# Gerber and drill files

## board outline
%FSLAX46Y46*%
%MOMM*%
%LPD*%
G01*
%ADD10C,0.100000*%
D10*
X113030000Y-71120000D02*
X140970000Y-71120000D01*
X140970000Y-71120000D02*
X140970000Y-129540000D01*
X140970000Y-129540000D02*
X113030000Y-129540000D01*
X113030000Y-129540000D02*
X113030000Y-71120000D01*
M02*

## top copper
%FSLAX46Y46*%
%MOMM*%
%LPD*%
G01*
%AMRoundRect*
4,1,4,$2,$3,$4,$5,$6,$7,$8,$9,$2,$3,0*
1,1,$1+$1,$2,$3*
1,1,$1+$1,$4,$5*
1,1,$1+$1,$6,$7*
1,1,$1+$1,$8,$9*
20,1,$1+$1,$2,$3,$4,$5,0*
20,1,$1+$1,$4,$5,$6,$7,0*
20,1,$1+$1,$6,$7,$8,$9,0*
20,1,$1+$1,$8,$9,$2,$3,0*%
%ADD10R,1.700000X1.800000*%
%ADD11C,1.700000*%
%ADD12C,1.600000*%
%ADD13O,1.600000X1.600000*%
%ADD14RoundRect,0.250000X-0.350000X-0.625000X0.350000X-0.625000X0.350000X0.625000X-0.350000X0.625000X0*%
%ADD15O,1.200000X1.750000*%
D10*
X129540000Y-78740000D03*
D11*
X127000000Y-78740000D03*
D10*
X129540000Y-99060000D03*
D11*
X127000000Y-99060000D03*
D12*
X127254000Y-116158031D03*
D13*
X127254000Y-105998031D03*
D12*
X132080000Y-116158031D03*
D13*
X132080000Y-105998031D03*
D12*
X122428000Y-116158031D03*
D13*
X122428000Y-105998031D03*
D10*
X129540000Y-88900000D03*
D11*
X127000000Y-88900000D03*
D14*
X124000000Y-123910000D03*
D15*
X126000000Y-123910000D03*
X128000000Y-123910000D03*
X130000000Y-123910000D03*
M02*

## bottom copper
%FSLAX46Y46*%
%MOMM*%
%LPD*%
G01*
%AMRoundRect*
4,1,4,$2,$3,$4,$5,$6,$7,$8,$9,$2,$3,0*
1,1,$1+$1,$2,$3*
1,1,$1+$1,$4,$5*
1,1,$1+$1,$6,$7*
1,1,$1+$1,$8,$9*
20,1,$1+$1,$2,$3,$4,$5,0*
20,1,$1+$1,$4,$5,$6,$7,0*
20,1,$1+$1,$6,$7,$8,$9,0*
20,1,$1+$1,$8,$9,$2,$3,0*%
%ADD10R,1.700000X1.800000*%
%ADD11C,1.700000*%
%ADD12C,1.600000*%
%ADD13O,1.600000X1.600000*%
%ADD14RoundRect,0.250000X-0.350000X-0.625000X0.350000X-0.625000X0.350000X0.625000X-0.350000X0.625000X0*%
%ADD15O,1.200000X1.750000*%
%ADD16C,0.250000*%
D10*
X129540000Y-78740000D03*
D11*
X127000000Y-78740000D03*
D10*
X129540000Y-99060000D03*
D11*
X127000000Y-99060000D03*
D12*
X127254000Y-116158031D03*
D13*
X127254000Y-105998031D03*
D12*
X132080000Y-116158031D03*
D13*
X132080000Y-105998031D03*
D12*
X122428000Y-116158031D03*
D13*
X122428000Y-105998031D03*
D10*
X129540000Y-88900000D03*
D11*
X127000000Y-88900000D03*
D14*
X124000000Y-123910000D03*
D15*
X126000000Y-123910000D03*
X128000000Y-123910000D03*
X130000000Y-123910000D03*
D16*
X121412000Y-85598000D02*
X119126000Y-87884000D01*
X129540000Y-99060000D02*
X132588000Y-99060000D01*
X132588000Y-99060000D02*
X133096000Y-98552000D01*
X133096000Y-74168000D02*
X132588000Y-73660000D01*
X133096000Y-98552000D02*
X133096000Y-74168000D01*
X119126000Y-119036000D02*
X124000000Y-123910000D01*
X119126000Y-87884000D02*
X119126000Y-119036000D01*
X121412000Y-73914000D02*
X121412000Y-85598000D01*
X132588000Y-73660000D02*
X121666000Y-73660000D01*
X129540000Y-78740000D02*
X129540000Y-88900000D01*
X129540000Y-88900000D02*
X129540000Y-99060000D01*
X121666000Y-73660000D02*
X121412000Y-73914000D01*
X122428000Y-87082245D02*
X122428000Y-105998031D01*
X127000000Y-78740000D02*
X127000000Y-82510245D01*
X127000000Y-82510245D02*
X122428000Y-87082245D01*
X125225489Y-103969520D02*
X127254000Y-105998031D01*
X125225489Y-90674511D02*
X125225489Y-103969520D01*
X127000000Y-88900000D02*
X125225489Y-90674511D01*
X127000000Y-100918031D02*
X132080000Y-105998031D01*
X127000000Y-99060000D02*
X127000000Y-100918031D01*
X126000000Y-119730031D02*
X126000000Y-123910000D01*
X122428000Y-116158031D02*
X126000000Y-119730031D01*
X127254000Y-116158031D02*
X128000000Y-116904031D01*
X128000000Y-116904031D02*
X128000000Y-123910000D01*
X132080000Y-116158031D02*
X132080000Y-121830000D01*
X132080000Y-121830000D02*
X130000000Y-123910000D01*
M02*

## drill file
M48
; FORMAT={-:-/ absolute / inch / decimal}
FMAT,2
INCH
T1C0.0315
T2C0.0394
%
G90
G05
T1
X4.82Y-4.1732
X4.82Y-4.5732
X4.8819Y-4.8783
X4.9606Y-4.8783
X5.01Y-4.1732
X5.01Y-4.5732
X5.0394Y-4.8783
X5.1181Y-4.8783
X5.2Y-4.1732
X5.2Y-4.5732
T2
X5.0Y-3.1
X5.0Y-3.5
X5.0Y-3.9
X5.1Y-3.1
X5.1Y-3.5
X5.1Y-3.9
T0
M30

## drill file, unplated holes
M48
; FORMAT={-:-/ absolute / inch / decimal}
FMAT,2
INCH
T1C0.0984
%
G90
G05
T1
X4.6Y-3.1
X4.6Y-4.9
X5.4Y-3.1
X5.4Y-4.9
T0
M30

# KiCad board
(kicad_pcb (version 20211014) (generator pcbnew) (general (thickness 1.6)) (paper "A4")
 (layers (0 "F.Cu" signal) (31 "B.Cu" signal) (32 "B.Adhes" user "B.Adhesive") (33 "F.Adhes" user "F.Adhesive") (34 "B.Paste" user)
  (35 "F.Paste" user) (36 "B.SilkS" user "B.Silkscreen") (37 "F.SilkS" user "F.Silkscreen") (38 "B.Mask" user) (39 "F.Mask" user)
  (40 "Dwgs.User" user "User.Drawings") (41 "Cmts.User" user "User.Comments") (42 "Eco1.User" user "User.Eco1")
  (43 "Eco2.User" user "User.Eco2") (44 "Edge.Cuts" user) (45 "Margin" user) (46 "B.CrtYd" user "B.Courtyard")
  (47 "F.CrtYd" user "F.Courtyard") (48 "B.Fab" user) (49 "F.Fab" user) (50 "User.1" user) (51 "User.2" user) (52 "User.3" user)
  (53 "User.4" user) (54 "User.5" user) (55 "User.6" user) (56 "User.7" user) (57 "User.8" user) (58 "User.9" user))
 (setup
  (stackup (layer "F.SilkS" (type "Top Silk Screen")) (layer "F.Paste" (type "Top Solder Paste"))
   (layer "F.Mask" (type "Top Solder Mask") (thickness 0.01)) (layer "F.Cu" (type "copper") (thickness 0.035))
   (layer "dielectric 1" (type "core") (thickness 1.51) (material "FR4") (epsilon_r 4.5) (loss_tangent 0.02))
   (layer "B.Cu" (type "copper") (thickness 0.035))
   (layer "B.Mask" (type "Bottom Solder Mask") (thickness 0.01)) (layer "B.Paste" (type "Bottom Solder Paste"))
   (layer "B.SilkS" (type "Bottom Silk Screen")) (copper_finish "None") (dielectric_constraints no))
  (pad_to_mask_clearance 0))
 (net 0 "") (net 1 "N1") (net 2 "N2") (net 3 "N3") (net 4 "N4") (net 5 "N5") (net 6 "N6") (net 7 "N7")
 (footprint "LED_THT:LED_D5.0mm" (layer "F.Cu") (at 129.54 78.74 180)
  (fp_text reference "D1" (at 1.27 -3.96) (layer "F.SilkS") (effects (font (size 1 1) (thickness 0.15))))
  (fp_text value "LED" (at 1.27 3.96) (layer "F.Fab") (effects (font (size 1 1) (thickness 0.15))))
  (pad "1" thru_hole rect (at 0 0 180) (size 1.7 1.8) (drill 1) (layers *.Cu *.Mask) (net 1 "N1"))
  (pad "2" thru_hole circle (at 2.54 0 180) (size 1.7 1.7) (drill 1) (layers *.Cu *.Mask) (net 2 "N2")))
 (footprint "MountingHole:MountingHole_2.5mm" (layer "F.Cu") (at 137.16 124.46)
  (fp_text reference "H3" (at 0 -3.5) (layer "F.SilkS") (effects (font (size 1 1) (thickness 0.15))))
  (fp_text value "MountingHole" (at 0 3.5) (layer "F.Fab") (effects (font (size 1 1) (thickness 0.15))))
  (pad "" np_thru_hole circle (at 0 0) (size 2.5 2.5) (drill 2.5) (layers *.Cu *.Mask)))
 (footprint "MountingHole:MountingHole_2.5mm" (layer "F.Cu") (at 137.16 78.74)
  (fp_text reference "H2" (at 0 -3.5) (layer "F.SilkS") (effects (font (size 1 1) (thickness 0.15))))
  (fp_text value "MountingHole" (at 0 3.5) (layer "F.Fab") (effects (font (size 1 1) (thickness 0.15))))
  (pad "" np_thru_hole circle (at 0 0) (size 2.5 2.5) (drill 2.5) (layers *.Cu *.Mask)))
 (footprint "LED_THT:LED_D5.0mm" (layer "F.Cu") (at 129.54 99.06 180)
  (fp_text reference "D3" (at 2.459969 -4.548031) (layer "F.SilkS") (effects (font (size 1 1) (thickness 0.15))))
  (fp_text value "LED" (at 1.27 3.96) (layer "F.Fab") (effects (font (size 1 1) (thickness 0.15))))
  (pad "1" thru_hole rect (at 0 0 180) (size 1.7 1.8) (drill 1) (layers *.Cu *.Mask) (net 1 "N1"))
  (pad "2" thru_hole circle (at 2.54 0 180) (size 1.7 1.7) (drill 1) (layers *.Cu *.Mask) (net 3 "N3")))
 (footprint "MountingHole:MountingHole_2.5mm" (layer "F.Cu") (at 116.84 124.46)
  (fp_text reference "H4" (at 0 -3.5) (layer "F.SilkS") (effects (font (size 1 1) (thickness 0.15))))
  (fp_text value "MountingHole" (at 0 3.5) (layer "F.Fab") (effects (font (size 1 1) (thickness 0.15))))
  (pad "" np_thru_hole circle (at 0 0) (size 2.5 2.5) (drill 2.5) (layers *.Cu *.Mask)))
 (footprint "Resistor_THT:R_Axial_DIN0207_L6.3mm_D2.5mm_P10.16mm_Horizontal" (layer "F.Cu") (at 127.254 116.158031 90)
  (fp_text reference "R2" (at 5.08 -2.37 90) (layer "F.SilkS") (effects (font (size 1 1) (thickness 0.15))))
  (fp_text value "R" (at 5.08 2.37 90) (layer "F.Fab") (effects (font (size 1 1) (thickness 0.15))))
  (pad "1" thru_hole circle (at 0 0 90) (size 1.6 1.6) (drill 0.8) (layers *.Cu *.Mask) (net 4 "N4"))
  (pad "2" thru_hole oval (at 10.16 0 90) (size 1.6 1.6) (drill 0.8) (layers *.Cu *.Mask) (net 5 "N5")))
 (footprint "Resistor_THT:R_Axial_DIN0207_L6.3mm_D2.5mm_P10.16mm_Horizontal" (layer "F.Cu") (at 132.08 116.158031 90)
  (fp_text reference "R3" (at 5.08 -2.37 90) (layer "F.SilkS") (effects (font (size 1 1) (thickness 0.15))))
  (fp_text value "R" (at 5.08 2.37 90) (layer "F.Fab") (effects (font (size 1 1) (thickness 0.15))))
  (pad "1" thru_hole circle (at 0 0 90) (size 1.6 1.6) (drill 0.8) (layers *.Cu *.Mask) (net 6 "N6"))
  (pad "2" thru_hole oval (at 10.16 0 90) (size 1.6 1.6) (drill 0.8) (layers *.Cu *.Mask) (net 3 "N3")))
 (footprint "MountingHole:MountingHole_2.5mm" (layer "F.Cu") (at 116.84 78.74)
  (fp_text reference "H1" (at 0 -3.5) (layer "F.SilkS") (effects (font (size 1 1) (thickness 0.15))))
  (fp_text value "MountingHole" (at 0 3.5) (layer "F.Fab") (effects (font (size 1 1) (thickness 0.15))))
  (pad "" np_thru_hole circle (at 0 0) (size 2.5 2.5) (drill 2.5) (layers *.Cu *.Mask)))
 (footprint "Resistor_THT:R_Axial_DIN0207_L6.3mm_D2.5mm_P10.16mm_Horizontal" (layer "F.Cu") (at 122.428 116.158031 90)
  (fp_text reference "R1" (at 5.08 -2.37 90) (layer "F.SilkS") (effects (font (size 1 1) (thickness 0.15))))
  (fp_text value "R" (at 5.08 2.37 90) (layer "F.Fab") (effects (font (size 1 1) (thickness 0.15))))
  (pad "1" thru_hole circle (at 0 0 90) (size 1.6 1.6) (drill 0.8) (layers *.Cu *.Mask) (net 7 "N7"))
  (pad "2" thru_hole oval (at 10.16 0 90) (size 1.6 1.6) (drill 0.8) (layers *.Cu *.Mask) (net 2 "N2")))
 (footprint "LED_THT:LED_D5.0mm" (layer "F.Cu") (at 129.54 88.9 180)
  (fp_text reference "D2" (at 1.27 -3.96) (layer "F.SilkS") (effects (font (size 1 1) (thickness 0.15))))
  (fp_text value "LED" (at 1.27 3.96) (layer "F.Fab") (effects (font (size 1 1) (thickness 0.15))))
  (pad "1" thru_hole rect (at 0 0 180) (size 1.7 1.8) (drill 1) (layers *.Cu *.Mask) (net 1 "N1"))
  (pad "2" thru_hole circle (at 2.54 0 180) (size 1.7 1.7) (drill 1) (layers *.Cu *.Mask) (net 5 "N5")))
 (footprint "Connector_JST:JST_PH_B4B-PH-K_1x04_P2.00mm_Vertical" (layer "F.Cu") (at 124 123.91)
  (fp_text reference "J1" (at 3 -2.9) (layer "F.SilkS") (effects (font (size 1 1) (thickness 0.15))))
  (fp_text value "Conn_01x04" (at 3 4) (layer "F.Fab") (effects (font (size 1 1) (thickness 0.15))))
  (pad "1" thru_hole roundrect (at 0 0) (size 1.2 1.75) (drill 0.8) (layers *.Cu *.Mask) (roundrect_rratio 0.2083333333) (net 1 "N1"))
  (pad "2" thru_hole oval (at 2 0) (size 1.2 1.75) (drill 0.8) (layers *.Cu *.Mask) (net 7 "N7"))
  (pad "3" thru_hole oval (at 4 0) (size 1.2 1.75) (drill 0.8) (layers *.Cu *.Mask) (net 4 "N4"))
  (pad "4" thru_hole oval (at 6 0) (size 1.2 1.75) (drill 0.8) (layers *.Cu *.Mask) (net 6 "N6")))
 (gr_rect (start 113.03 71.12) (end 140.97 129.54) (layer "Edge.Cuts") (width 0.1) (fill none))
 (segment (start 121.412 85.598) (end 119.126 87.884) (width 0.25) (layer "B.Cu") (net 1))
 (segment (start 129.54 99.06) (end 132.588 99.06) (width 0.25) (layer "B.Cu") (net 1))
 (segment (start 132.588 99.06) (end 133.096 98.552) (width 0.25) (layer "B.Cu") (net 1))
 (segment (start 133.096 74.168) (end 132.588 73.66) (width 0.25) (layer "B.Cu") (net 1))
 (segment (start 133.096 98.552) (end 133.096 74.168) (width 0.25) (layer "B.Cu") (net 1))
 (segment (start 119.126 119.036) (end 124 123.91) (width 0.25) (layer "B.Cu") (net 1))
 (segment (start 119.126 87.884) (end 119.126 119.036) (width 0.25) (layer "B.Cu") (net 1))
 (segment (start 121.412 73.914) (end 121.412 85.598) (width 0.25) (layer "B.Cu") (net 1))
 (segment (start 132.588 73.66) (end 121.666 73.66) (width 0.25) (layer "B.Cu") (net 1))
 (segment (start 129.54 78.74) (end 129.54 88.9) (width 0.25) (layer "B.Cu") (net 1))
 (segment (start 129.54 88.9) (end 129.54 99.06) (width 0.25) (layer "B.Cu") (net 1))
 (segment (start 121.666 73.66) (end 121.412 73.914) (width 0.25) (layer "B.Cu") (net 1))
 (segment (start 122.428 87.082245) (end 122.428 105.998031) (width 0.25) (layer "B.Cu") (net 2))
 (segment (start 127 78.74) (end 127 82.510245) (width 0.25) (layer "B.Cu") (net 2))
 (segment (start 127 82.510245) (end 122.428 87.082245) (width 0.25) (layer "B.Cu") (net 2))
 (segment (start 125.225489 103.96952) (end 127.254 105.998031) (width 0.25) (layer "B.Cu") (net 5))
 (segment (start 125.225489 90.674511) (end 125.225489 103.96952) (width 0.25) (layer "B.Cu") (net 5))
 (segment (start 127 88.9) (end 125.225489 90.674511) (width 0.25) (layer "B.Cu") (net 5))
 (segment (start 127 100.918031) (end 132.08 105.998031) (width 0.25) (layer "B.Cu") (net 3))
 (segment (start 127 99.06) (end 127 100.918031) (width 0.25) (layer "B.Cu") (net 3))
 (segment (start 126 119.730031) (end 126 123.91) (width 0.25) (layer "B.Cu") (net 7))
 (segment (start 122.428 116.158031) (end 126 119.730031) (width 0.25) (layer "B.Cu") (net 7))
 (segment (start 127.254 116.158031) (end 128 116.904031) (width 0.25) (layer "B.Cu") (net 4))
 (segment (start 128 116.904031) (end 128 123.91) (width 0.25) (layer "B.Cu") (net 4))
 (segment (start 132.08 116.158031) (end 132.08 121.83) (width 0.25) (layer "B.Cu") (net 6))
 (segment (start 132.08 121.83) (end 130 123.91) (width 0.25) (layer "B.Cu") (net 6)))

